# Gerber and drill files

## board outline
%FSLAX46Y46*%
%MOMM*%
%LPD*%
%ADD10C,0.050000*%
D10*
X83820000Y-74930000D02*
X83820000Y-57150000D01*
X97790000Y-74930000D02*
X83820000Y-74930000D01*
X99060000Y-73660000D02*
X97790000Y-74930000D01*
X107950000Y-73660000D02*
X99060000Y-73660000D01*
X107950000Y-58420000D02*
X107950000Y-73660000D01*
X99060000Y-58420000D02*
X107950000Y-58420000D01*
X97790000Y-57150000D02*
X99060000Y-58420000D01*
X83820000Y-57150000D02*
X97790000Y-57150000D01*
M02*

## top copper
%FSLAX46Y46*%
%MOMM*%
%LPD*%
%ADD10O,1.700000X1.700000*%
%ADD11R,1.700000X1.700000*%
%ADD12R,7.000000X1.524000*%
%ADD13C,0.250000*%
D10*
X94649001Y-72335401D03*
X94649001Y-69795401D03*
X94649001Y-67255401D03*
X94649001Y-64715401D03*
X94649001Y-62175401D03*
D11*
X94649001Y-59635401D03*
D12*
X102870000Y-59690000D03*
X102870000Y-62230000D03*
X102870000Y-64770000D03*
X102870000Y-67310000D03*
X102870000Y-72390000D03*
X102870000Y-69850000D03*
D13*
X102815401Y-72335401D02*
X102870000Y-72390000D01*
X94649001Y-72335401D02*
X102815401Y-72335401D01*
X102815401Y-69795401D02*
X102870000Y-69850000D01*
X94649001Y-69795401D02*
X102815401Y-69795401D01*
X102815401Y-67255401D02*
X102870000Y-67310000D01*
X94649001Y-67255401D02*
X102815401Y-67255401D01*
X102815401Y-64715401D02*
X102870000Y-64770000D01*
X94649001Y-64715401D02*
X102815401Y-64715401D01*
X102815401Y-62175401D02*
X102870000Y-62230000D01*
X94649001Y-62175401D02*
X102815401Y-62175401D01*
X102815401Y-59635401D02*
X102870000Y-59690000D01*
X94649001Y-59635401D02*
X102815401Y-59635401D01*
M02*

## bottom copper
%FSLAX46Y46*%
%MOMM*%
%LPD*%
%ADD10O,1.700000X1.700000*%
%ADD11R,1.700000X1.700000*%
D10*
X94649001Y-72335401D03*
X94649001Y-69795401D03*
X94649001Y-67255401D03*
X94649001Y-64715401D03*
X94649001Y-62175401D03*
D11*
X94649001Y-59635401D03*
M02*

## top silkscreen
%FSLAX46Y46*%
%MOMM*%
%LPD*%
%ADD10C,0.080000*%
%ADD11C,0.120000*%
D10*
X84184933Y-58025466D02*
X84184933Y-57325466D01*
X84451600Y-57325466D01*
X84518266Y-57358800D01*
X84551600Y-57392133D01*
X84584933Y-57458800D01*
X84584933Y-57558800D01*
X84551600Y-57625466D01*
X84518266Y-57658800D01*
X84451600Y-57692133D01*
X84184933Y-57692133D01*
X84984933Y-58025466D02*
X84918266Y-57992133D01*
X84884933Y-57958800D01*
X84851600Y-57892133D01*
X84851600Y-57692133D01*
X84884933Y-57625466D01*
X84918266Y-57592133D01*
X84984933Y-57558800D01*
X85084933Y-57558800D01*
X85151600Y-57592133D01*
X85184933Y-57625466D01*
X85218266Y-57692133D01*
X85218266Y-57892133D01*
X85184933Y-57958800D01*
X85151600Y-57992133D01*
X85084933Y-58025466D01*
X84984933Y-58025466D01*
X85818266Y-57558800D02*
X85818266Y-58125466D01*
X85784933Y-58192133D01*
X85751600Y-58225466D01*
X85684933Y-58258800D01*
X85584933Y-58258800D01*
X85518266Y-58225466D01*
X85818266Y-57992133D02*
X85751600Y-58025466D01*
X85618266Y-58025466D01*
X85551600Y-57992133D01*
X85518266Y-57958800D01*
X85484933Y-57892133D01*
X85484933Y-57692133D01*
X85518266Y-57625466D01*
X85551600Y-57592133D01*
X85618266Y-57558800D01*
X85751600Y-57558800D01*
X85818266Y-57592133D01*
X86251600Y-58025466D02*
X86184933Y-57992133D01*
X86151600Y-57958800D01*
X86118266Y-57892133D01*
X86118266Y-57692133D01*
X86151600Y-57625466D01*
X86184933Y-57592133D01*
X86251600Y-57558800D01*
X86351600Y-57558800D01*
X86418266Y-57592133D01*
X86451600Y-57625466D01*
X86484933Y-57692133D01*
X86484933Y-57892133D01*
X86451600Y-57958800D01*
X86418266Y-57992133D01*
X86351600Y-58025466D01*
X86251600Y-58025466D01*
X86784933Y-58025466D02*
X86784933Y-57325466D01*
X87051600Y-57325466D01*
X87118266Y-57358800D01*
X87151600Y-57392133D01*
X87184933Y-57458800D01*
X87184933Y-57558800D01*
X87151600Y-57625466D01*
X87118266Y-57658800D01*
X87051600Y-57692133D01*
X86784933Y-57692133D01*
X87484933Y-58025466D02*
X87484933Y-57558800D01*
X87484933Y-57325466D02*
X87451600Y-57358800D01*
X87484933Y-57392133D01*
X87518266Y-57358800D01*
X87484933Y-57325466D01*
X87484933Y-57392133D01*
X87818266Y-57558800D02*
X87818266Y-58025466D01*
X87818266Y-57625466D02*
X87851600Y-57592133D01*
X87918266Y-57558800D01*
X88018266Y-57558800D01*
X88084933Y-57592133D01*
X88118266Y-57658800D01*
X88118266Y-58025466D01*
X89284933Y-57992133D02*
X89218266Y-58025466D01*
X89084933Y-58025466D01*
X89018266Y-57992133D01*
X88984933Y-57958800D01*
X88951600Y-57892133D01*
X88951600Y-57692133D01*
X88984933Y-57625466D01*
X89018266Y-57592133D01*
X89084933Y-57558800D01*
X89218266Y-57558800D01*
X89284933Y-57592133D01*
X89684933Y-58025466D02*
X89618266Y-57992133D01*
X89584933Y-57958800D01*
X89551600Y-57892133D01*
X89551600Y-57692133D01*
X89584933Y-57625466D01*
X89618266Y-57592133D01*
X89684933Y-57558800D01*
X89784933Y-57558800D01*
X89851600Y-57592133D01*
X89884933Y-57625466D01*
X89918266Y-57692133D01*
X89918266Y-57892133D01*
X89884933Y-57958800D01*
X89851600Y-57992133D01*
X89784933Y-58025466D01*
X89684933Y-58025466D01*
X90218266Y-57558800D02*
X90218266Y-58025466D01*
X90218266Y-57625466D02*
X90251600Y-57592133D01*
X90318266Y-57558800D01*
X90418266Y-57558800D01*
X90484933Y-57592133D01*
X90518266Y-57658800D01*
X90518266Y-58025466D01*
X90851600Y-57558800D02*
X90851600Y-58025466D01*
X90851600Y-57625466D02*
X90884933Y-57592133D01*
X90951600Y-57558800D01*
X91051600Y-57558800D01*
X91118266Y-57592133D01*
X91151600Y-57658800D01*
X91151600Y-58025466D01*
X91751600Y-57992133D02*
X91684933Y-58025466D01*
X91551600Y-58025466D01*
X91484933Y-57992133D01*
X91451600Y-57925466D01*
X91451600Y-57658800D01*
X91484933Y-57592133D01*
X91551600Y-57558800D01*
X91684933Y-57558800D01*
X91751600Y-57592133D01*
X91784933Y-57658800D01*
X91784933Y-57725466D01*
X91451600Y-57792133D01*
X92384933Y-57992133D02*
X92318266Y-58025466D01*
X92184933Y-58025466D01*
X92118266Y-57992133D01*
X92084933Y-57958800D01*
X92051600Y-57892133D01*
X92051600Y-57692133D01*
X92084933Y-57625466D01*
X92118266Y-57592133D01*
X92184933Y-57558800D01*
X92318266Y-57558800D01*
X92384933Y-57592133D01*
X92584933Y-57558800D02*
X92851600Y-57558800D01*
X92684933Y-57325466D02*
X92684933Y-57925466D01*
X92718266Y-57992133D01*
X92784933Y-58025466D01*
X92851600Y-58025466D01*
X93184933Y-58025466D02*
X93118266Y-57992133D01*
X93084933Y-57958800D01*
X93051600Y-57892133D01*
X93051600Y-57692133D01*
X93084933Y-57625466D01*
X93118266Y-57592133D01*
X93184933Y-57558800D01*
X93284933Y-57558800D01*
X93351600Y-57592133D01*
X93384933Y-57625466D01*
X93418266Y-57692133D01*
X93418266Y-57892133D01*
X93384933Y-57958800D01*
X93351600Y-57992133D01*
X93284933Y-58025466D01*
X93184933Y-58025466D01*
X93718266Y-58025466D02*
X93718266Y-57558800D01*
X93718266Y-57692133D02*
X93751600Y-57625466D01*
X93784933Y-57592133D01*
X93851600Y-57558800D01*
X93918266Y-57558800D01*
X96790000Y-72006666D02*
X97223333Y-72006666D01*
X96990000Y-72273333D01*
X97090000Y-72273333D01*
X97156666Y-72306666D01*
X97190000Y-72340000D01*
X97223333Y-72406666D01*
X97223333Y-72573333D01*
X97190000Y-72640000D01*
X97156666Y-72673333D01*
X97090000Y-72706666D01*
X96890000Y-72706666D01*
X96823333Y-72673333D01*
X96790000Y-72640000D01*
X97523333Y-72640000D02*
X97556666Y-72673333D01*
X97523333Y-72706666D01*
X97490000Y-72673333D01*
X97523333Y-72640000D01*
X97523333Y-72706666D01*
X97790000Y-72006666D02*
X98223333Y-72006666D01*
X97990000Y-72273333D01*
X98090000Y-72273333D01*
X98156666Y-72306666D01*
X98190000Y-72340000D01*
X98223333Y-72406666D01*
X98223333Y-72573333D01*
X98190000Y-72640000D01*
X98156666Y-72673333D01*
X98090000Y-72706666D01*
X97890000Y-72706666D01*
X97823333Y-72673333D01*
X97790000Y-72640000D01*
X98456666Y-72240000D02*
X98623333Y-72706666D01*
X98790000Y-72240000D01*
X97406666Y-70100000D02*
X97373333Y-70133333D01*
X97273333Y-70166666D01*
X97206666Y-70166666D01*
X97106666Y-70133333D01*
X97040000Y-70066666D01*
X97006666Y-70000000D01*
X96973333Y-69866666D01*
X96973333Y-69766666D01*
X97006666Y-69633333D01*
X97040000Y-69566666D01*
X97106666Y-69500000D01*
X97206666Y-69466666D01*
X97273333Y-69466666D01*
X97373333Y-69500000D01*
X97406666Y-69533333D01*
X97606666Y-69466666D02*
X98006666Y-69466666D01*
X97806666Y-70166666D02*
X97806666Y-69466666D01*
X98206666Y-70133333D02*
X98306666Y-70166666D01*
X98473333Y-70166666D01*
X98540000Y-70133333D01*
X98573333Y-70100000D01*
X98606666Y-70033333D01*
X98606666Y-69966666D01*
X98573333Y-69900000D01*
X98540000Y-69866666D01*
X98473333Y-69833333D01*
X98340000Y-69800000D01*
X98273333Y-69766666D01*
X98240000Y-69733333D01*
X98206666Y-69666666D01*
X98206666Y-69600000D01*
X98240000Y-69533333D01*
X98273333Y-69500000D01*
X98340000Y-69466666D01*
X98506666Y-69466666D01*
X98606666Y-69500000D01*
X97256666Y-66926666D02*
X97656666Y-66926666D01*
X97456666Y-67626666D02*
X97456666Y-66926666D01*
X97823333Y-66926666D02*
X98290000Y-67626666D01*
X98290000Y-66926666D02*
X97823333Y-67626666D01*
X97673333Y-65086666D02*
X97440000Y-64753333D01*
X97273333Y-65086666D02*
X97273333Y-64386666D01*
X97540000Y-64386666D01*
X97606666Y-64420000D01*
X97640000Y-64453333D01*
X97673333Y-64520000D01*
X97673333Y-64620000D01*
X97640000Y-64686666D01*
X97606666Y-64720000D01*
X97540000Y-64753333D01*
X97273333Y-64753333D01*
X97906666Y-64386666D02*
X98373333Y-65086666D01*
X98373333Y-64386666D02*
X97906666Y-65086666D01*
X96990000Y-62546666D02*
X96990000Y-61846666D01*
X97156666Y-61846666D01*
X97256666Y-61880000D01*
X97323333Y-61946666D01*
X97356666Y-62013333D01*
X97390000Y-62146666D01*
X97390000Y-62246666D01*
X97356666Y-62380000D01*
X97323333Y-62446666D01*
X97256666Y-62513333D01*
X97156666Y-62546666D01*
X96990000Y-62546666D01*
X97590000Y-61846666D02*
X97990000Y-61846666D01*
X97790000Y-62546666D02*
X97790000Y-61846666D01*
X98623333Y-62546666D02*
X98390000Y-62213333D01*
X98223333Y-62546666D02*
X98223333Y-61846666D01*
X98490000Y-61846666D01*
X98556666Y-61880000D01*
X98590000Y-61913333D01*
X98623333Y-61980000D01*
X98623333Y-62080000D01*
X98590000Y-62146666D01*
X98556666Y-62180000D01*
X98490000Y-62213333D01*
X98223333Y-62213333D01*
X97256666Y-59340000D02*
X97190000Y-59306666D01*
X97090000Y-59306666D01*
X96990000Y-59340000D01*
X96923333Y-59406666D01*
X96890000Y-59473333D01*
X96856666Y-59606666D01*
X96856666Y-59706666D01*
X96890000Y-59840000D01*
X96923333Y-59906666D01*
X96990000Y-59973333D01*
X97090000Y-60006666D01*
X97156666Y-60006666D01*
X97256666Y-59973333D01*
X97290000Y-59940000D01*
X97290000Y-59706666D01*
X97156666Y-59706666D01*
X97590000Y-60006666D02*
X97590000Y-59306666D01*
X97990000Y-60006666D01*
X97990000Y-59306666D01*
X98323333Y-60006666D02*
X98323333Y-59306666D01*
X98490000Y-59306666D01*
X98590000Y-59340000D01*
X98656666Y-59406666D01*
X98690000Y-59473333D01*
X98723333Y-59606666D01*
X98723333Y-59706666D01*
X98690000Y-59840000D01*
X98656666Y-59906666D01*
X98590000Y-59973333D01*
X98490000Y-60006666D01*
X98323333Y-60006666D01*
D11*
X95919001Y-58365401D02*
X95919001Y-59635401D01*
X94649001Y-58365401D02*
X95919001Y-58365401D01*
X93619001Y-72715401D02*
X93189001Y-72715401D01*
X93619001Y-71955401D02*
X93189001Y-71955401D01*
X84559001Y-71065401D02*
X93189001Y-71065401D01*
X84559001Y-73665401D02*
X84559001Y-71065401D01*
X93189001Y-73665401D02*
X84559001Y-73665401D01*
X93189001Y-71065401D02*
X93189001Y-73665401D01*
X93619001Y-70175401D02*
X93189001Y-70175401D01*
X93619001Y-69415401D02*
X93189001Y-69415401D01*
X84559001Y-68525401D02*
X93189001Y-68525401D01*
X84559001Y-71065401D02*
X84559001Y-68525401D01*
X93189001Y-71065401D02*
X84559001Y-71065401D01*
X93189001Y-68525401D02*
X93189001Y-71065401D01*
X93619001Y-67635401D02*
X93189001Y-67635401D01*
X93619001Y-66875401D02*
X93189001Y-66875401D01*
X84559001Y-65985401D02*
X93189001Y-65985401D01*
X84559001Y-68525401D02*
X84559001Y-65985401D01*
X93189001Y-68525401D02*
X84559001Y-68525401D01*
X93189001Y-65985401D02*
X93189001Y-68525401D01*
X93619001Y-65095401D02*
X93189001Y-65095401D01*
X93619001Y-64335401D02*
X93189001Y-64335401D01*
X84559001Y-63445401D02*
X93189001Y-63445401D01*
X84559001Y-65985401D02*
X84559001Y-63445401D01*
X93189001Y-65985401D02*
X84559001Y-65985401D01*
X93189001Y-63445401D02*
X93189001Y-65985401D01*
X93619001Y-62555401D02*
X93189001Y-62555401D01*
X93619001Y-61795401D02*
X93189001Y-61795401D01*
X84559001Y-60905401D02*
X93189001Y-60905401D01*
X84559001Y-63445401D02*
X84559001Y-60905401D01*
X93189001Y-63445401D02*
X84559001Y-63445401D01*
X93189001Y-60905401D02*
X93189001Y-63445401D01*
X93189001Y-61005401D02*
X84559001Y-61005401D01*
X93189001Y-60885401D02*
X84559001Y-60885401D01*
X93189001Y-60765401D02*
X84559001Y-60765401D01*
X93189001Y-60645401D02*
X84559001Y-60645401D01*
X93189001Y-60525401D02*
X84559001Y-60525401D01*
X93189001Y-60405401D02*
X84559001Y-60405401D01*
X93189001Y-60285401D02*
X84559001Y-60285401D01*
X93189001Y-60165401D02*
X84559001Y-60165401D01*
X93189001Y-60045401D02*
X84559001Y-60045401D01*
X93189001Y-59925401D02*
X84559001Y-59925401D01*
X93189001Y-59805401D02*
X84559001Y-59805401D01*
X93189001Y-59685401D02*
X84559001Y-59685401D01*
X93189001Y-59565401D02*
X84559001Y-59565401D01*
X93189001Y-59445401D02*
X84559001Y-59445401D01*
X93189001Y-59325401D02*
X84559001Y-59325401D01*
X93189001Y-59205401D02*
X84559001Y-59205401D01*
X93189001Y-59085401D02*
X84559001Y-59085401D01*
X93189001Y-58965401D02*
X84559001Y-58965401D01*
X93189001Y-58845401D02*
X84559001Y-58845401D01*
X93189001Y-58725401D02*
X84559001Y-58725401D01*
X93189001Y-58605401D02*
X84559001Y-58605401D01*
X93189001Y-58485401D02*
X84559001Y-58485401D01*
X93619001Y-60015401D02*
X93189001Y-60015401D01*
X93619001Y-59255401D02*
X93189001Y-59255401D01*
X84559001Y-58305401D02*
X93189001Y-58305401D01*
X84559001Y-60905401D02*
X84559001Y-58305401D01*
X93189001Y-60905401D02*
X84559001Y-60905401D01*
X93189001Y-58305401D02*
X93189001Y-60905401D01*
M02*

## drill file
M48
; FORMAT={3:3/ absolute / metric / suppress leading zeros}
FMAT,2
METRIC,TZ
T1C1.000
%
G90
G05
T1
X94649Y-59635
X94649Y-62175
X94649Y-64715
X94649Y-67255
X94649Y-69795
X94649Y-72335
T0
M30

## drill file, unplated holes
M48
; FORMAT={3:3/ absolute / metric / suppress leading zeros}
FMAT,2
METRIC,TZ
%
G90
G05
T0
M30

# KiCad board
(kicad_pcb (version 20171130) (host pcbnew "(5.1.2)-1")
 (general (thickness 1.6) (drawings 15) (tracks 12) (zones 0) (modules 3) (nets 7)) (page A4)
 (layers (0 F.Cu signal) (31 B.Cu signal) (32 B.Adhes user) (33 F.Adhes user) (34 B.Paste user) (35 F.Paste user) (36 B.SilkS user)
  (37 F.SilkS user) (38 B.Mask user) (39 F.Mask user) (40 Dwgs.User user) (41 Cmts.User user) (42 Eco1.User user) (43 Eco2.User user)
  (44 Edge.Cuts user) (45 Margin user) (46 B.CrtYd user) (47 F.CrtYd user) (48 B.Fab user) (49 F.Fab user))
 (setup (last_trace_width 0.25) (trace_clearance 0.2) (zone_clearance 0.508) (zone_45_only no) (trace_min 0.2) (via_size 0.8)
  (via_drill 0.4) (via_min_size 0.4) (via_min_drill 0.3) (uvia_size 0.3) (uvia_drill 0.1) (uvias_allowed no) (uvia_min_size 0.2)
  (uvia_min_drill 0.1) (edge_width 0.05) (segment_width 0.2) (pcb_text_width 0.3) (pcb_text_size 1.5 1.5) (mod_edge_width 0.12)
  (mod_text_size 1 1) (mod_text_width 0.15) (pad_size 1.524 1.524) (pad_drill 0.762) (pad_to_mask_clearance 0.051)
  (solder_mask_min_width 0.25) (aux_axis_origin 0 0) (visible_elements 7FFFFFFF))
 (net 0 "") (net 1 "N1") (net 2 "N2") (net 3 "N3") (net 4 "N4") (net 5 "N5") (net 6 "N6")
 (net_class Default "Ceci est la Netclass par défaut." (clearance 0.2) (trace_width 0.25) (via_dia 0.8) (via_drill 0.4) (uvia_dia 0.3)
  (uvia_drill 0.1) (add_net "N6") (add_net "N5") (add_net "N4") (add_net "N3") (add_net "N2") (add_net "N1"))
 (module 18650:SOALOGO (layer B.Cu) (at 88.9 66.04 270)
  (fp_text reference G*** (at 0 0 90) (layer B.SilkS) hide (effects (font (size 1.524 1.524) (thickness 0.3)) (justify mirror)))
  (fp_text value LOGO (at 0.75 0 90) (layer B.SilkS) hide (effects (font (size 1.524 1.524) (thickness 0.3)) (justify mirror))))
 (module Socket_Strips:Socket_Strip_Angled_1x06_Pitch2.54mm (layer F.Cu) (at 94.649001 59.635401)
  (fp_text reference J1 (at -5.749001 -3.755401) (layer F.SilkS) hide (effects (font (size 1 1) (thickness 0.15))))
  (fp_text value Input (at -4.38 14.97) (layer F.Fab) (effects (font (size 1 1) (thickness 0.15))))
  (fp_line (start 1.27 -1.27) (end 1.27 0) (layer F.SilkS) (width 0.12))
  (fp_line (start 0 -1.27) (end 1.27 -1.27) (layer F.SilkS) (width 0.12))
  (fp_line (start -1.03 13.08) (end -1.46 13.08) (layer F.SilkS) (width 0.12))
  (fp_line (start -1.03 12.32) (end -1.46 12.32) (layer F.SilkS) (width 0.12))
  (fp_line (start -10.09 11.43) (end -1.46 11.43) (layer F.SilkS) (width 0.12))
  (fp_line (start -10.09 14.03) (end -10.09 11.43) (layer F.SilkS) (width 0.12))
  (fp_line (start -1.46 14.03) (end -10.09 14.03) (layer F.SilkS) (width 0.12))
  (fp_line (start -1.46 11.43) (end -1.46 14.03) (layer F.SilkS) (width 0.12))
  (fp_line (start -1.03 10.54) (end -1.46 10.54) (layer F.SilkS) (width 0.12))
  (fp_line (start -1.03 9.78) (end -1.46 9.78) (layer F.SilkS) (width 0.12))
  (fp_line (start -10.09 8.89) (end -1.46 8.89) (layer F.SilkS) (width 0.12))
  (fp_line (start -10.09 11.43) (end -10.09 8.89) (layer F.SilkS) (width 0.12))
  (fp_line (start -1.46 11.43) (end -10.09 11.43) (layer F.SilkS) (width 0.12))
  (fp_line (start -1.46 8.89) (end -1.46 11.43) (layer F.SilkS) (width 0.12))
  (fp_line (start -1.03 8) (end -1.46 8) (layer F.SilkS) (width 0.12))
  (fp_line (start -1.03 7.24) (end -1.46 7.24) (layer F.SilkS) (width 0.12))
  (fp_line (start -10.09 6.35) (end -1.46 6.35) (layer F.SilkS) (width 0.12))
  (fp_line (start -10.09 8.89) (end -10.09 6.35) (layer F.SilkS) (width 0.12))
  (fp_line (start -1.46 8.89) (end -10.09 8.89) (layer F.SilkS) (width 0.12))
  (fp_line (start -1.46 6.35) (end -1.46 8.89) (layer F.SilkS) (width 0.12))
  (fp_line (start -1.03 5.46) (end -1.46 5.46) (layer F.SilkS) (width 0.12))
  (fp_line (start -1.03 4.7) (end -1.46 4.7) (layer F.SilkS) (width 0.12))
  (fp_line (start -10.09 3.81) (end -1.46 3.81) (layer F.SilkS) (width 0.12))
  (fp_line (start -10.09 6.35) (end -10.09 3.81) (layer F.SilkS) (width 0.12))
  (fp_line (start -1.46 6.35) (end -10.09 6.35) (layer F.SilkS) (width 0.12))
  (fp_line (start -1.46 3.81) (end -1.46 6.35) (layer F.SilkS) (width 0.12))
  (fp_line (start -1.03 2.92) (end -1.46 2.92) (layer F.SilkS) (width 0.12))
  (fp_line (start -1.03 2.16) (end -1.46 2.16) (layer F.SilkS) (width 0.12))
  (fp_line (start -10.09 1.27) (end -1.46 1.27) (layer F.SilkS) (width 0.12))
  (fp_line (start -10.09 3.81) (end -10.09 1.27) (layer F.SilkS) (width 0.12))
  (fp_line (start -1.46 3.81) (end -10.09 3.81) (layer F.SilkS) (width 0.12))
  (fp_line (start -1.46 1.27) (end -1.46 3.81) (layer F.SilkS) (width 0.12))
  (fp_line (start -1.46 1.37) (end -10.09 1.37) (layer F.SilkS) (width 0.12))
  (fp_line (start -1.46 1.25) (end -10.09 1.25) (layer F.SilkS) (width 0.12))
  (fp_line (start -1.46 1.13) (end -10.09 1.13) (layer F.SilkS) (width 0.12))
  (fp_line (start -1.46 1.01) (end -10.09 1.01) (layer F.SilkS) (width 0.12))
  (fp_line (start -1.46 0.89) (end -10.09 0.89) (layer F.SilkS) (width 0.12))
  (fp_line (start -1.46 0.77) (end -10.09 0.77) (layer F.SilkS) (width 0.12))
  (fp_line (start -1.46 0.65) (end -10.09 0.65) (layer F.SilkS) (width 0.12))
  (fp_line (start -1.46 0.53) (end -10.09 0.53) (layer F.SilkS) (width 0.12))
  (fp_line (start -1.46 0.41) (end -10.09 0.41) (layer F.SilkS) (width 0.12))
  (fp_line (start -1.46 0.29) (end -10.09 0.29) (layer F.SilkS) (width 0.12))
  (fp_line (start -1.46 0.17) (end -10.09 0.17) (layer F.SilkS) (width 0.12))
  (fp_line (start -1.46 0.05) (end -10.09 0.05) (layer F.SilkS) (width 0.12))
  (fp_line (start -1.46 -0.07) (end -10.09 -0.07) (layer F.SilkS) (width 0.12))
  (fp_line (start -1.46 -0.19) (end -10.09 -0.19) (layer F.SilkS) (width 0.12))
  (fp_line (start -1.46 -0.31) (end -10.09 -0.31) (layer F.SilkS) (width 0.12))
  (fp_line (start -1.46 -0.43) (end -10.09 -0.43) (layer F.SilkS) (width 0.12))
  (fp_line (start -1.46 -0.55) (end -10.09 -0.55) (layer F.SilkS) (width 0.12))
  (fp_line (start -1.46 -0.67) (end -10.09 -0.67) (layer F.SilkS) (width 0.12))
  (fp_line (start -1.46 -0.79) (end -10.09 -0.79) (layer F.SilkS) (width 0.12))
  (fp_line (start -1.46 -0.91) (end -10.09 -0.91) (layer F.SilkS) (width 0.12))
  (fp_line (start -1.46 -1.03) (end -10.09 -1.03) (layer F.SilkS) (width 0.12))
  (fp_line (start -1.46 -1.15) (end -10.09 -1.15) (layer F.SilkS) (width 0.12))
  (fp_line (start -1.03 0.38) (end -1.46 0.38) (layer F.SilkS) (width 0.12))
  (fp_line (start -1.03 -0.38) (end -1.46 -0.38) (layer F.SilkS) (width 0.12))
  (fp_line (start -10.09 -1.33) (end -1.46 -1.33) (layer F.SilkS) (width 0.12))
  (fp_line (start -10.09 1.27) (end -10.09 -1.33) (layer F.SilkS) (width 0.12))
  (fp_line (start -1.46 1.27) (end -10.09 1.27) (layer F.SilkS) (width 0.12))
  (fp_line (start -1.46 -1.33) (end -1.46 1.27) (layer F.SilkS) (width 0.12))
  (pad 6 thru_hole oval (at 0 12.7) (size 1.7 1.7) (drill 1) (layers *.Cu *.Mask) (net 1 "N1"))
  (pad 5 thru_hole oval (at 0 10.16) (size 1.7 1.7) (drill 1) (layers *.Cu *.Mask) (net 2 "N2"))
  (pad 4 thru_hole oval (at 0 7.62) (size 1.7 1.7) (drill 1) (layers *.Cu *.Mask) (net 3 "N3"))
  (pad 3 thru_hole oval (at 0 5.08) (size 1.7 1.7) (drill 1) (layers *.Cu *.Mask) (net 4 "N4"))
  (pad 2 thru_hole oval (at 0 2.54) (size 1.7 1.7) (drill 1) (layers *.Cu *.Mask) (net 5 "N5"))
  (pad 1 thru_hole rect (at 0 0) (size 1.7 1.7) (drill 1) (layers *.Cu *.Mask) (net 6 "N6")))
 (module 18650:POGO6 (layer F.Cu) (at 99.06 58.42 270)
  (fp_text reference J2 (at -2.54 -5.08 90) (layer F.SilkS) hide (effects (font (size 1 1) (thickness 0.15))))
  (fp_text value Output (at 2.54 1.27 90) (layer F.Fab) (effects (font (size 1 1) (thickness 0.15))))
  (pad 1 smd rect (at 1.27 -3.81 270) (size 1.524 7) (layers F.Cu F.Paste F.Mask) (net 6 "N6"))
  (pad 2 smd rect (at 3.81 -3.81 270) (size 1.524 7) (layers F.Cu F.Paste F.Mask) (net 5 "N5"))
  (pad 3 smd rect (at 6.35 -3.81 270) (size 1.524 7) (layers F.Cu F.Paste F.Mask) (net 4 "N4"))
  (pad 4 smd rect (at 8.89 -3.81 270) (size 1.524 7) (layers F.Cu F.Paste F.Mask) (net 3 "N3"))
  (pad 6 smd rect (at 13.97 -3.81 270) (size 1.524 7) (layers F.Cu F.Paste F.Mask) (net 1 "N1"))
  (pad 5 smd rect (at 11.43 -3.81 270) (size 1.524 7) (layers F.Cu F.Paste F.Mask) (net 2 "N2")))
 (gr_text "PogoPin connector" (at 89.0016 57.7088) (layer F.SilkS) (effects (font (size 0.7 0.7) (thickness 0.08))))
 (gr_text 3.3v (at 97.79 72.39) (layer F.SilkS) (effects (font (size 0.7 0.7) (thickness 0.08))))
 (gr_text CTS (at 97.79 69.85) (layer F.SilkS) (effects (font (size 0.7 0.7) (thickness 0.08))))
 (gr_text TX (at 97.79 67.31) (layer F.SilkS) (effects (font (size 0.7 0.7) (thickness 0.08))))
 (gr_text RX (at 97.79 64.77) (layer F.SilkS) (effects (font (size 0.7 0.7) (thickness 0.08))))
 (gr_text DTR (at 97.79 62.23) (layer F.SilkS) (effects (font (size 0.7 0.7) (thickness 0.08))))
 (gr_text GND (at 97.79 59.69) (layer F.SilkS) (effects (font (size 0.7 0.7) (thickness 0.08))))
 (gr_line (start 83.82 74.93) (end 83.82 57.15) (layer Edge.Cuts) (width 0.05))
 (gr_line (start 97.79 74.93) (end 83.82 74.93) (layer Edge.Cuts) (width 0.05))
 (gr_line (start 99.06 73.66) (end 97.79 74.93) (layer Edge.Cuts) (width 0.05))
 (gr_line (start 107.95 73.66) (end 99.06 73.66) (layer Edge.Cuts) (width 0.05))
 (gr_line (start 107.95 58.42) (end 107.95 73.66) (layer Edge.Cuts) (width 0.05))
 (gr_line (start 99.06 58.42) (end 107.95 58.42) (layer Edge.Cuts) (width 0.05))
 (gr_line (start 97.79 57.15) (end 99.06 58.42) (layer Edge.Cuts) (width 0.05))
 (gr_line (start 83.82 57.15) (end 97.79 57.15) (layer Edge.Cuts) (width 0.05))
 (segment (start 102.815401 72.335401) (end 102.87 72.39) (width 0.25) (layer F.Cu) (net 1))
 (segment (start 94.649001 72.335401) (end 102.815401 72.335401) (width 0.25) (layer F.Cu) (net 1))
 (segment (start 102.815401 69.795401) (end 102.87 69.85) (width 0.25) (layer F.Cu) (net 2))
 (segment (start 94.649001 69.795401) (end 102.815401 69.795401) (width 0.25) (layer F.Cu) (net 2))
 (segment (start 102.815401 67.255401) (end 102.87 67.31) (width 0.25) (layer F.Cu) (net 3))
 (segment (start 94.649001 67.255401) (end 102.815401 67.255401) (width 0.25) (layer F.Cu) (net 3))
 (segment (start 102.815401 64.715401) (end 102.87 64.77) (width 0.25) (layer F.Cu) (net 4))
 (segment (start 94.649001 64.715401) (end 102.815401 64.715401) (width 0.25) (layer F.Cu) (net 4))
 (segment (start 102.815401 62.175401) (end 102.87 62.23) (width 0.25) (layer F.Cu) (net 5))
 (segment (start 94.649001 62.175401) (end 102.815401 62.175401) (width 0.25) (layer F.Cu) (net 5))
 (segment (start 102.815401 59.635401) (end 102.87 59.69) (width 0.25) (layer F.Cu) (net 6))
 (segment (start 94.649001 59.635401) (end 102.815401 59.635401) (width 0.25) (layer F.Cu) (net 6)))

